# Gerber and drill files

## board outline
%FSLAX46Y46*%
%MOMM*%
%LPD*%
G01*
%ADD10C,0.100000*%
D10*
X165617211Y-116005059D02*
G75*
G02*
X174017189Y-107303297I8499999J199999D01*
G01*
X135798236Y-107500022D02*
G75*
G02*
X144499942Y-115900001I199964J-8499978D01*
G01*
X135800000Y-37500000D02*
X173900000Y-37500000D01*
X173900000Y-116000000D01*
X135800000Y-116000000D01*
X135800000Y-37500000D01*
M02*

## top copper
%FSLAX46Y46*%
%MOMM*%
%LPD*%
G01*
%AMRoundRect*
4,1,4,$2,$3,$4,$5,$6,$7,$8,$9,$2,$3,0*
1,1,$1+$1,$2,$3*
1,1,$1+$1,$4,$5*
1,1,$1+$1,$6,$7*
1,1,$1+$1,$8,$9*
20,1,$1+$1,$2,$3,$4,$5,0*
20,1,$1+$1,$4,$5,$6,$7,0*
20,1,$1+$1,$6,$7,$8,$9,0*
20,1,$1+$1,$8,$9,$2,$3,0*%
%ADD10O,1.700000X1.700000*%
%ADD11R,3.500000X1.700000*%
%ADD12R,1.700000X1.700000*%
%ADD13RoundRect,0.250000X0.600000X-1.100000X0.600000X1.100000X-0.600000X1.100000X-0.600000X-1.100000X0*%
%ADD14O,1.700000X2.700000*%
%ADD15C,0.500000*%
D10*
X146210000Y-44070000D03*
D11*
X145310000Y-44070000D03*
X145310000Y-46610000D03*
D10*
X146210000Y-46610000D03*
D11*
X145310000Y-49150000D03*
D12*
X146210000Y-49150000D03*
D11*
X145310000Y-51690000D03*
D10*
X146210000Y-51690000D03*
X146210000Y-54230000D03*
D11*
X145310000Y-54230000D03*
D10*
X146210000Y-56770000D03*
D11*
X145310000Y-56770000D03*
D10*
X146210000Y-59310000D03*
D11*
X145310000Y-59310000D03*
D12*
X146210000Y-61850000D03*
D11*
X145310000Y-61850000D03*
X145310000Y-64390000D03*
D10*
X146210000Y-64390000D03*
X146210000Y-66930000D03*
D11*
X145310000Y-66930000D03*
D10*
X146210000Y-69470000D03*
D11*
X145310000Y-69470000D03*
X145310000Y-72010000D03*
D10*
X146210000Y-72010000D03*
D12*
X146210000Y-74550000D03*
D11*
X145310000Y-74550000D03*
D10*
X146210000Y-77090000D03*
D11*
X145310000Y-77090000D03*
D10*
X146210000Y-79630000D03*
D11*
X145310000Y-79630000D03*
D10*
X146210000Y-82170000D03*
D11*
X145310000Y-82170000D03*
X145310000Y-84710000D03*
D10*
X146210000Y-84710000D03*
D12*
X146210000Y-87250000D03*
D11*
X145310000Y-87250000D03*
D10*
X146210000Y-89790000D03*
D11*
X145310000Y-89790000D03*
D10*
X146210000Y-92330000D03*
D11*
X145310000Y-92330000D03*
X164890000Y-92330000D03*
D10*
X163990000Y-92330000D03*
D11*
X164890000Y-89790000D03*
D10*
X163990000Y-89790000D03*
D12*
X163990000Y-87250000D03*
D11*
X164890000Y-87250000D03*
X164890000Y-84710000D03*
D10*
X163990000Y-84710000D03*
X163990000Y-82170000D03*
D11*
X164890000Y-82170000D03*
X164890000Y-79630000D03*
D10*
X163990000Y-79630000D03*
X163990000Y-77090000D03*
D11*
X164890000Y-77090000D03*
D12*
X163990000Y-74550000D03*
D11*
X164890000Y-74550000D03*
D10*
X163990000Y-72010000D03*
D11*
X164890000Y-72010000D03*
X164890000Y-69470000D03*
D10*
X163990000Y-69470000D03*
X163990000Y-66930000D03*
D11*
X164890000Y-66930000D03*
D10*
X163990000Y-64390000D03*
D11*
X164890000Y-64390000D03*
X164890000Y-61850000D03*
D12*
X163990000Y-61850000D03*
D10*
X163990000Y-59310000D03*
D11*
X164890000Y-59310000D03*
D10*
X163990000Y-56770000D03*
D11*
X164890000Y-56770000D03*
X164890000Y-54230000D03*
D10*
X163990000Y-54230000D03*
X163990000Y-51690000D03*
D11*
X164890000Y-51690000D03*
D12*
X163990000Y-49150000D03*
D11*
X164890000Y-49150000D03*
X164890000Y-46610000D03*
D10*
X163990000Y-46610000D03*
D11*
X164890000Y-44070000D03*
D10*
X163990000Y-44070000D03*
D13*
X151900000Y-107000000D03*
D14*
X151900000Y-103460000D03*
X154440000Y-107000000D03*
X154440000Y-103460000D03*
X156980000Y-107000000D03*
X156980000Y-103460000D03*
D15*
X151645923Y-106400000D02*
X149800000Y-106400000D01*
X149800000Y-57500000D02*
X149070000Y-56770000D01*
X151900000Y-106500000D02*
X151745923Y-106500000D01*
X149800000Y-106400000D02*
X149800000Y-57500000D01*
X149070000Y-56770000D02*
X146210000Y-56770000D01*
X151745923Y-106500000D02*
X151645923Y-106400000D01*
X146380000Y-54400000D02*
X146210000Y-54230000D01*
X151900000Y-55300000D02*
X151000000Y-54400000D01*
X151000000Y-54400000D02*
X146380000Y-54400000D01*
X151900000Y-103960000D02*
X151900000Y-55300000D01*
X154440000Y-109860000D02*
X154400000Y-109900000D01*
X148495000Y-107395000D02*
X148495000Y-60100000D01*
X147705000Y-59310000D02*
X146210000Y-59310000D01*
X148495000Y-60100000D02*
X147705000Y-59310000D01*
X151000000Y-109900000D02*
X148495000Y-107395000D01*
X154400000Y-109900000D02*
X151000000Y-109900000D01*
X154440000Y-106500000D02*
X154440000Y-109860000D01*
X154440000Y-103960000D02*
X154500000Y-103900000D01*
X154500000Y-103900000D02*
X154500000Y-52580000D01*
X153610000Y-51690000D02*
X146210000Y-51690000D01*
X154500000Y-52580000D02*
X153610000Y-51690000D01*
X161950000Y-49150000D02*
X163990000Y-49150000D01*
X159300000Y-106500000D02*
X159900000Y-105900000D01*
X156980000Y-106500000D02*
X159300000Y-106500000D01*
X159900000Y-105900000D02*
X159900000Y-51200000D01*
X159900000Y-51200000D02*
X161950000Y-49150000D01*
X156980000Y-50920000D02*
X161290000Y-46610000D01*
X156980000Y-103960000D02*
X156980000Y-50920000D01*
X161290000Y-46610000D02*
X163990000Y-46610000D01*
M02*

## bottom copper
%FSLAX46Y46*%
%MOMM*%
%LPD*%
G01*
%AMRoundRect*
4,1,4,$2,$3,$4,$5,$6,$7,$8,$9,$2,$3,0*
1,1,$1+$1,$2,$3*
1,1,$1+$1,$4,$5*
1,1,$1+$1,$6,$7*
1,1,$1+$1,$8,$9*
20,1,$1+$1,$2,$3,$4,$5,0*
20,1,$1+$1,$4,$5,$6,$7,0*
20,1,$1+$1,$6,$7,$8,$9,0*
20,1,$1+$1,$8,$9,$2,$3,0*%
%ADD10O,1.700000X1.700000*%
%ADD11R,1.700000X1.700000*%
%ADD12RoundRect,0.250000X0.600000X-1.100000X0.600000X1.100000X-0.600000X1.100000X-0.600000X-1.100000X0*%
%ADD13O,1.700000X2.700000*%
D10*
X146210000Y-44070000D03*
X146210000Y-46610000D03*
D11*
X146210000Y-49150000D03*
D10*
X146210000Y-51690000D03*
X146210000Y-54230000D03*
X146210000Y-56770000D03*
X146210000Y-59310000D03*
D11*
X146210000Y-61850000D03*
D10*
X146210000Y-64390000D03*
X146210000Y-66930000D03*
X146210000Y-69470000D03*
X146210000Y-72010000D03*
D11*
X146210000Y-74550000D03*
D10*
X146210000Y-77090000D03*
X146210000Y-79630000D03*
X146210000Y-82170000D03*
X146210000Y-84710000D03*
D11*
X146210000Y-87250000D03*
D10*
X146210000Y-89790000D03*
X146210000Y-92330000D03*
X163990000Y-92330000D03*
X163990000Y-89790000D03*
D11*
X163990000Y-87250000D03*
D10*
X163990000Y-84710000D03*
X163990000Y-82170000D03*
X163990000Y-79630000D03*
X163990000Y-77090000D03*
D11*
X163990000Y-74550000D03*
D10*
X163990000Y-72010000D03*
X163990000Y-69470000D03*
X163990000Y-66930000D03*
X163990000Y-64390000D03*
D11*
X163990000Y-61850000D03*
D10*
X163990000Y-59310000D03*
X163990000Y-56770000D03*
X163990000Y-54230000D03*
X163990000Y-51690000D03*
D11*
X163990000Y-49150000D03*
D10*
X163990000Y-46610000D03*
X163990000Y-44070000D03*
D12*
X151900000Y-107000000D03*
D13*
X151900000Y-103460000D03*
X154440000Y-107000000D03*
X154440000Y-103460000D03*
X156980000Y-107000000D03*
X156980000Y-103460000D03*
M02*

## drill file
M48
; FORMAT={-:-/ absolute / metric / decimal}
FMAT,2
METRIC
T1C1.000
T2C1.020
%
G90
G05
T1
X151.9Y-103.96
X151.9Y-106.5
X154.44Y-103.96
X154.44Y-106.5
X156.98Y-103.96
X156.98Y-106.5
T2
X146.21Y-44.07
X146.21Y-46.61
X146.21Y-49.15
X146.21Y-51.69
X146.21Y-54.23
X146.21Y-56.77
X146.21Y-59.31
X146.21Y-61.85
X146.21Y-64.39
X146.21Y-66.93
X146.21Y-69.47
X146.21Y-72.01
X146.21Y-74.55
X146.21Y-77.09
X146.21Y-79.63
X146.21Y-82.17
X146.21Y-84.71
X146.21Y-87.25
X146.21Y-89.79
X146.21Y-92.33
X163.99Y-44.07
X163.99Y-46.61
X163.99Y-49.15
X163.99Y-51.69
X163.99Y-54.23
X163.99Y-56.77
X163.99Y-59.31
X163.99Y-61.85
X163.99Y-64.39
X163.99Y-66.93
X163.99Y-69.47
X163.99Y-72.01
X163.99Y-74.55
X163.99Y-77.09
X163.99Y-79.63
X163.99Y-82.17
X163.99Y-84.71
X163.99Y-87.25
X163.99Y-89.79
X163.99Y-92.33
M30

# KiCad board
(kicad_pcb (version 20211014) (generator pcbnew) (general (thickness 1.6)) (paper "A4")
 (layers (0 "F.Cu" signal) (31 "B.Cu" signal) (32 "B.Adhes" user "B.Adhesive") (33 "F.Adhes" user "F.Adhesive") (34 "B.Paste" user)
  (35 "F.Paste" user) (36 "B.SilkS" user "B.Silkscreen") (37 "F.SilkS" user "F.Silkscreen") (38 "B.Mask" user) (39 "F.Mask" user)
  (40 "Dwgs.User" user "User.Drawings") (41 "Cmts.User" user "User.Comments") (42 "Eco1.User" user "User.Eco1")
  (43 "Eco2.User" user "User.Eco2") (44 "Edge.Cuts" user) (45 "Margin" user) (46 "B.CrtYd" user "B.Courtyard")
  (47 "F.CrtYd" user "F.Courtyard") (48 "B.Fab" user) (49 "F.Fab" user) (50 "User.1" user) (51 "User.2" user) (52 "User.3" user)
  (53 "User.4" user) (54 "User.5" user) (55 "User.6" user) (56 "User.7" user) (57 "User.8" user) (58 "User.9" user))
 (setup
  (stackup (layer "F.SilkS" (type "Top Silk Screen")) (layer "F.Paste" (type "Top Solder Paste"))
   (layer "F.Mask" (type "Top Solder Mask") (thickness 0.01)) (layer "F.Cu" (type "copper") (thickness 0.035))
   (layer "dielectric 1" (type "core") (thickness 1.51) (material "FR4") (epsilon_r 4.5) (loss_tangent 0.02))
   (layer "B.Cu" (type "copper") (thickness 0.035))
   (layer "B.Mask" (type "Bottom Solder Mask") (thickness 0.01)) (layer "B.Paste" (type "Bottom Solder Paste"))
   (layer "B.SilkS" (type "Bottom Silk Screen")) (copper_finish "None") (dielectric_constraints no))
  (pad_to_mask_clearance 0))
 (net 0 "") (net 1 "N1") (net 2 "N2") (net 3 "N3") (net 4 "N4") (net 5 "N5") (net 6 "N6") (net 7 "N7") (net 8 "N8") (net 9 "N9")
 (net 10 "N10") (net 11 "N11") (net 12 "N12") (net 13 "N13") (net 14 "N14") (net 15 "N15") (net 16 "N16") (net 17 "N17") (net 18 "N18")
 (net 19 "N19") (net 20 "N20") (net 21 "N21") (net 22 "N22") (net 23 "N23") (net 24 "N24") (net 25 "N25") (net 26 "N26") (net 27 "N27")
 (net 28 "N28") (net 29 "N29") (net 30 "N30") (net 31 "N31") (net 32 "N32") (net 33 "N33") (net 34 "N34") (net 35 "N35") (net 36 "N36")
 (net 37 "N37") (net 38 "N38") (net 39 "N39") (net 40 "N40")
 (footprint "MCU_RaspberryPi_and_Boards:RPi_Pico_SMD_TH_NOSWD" (layer "F.Cu") (at 155.1 68.2)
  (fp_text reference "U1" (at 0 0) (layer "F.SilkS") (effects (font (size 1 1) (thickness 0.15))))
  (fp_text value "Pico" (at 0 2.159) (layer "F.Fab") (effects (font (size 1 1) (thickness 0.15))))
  (pad "1" thru_hole oval (at -8.89 -24.13) (size 1.7 1.7) (drill 1.02) (layers *.Cu *.Mask) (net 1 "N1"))
  (pad "1" smd rect (at -8.89 -24.13) (size 3.5 1.7) (drill (offset -0.9 0)) (layers "F.Cu" "F.Mask") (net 1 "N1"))
  (pad "2" smd rect (at -8.89 -21.59) (size 3.5 1.7) (drill (offset -0.9 0)) (layers "F.Cu" "F.Mask") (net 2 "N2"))
  (pad "2" thru_hole oval (at -8.89 -21.59) (size 1.7 1.7) (drill 1.02) (layers *.Cu *.Mask) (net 2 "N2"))
  (pad "3" smd rect (at -8.89 -19.05) (size 3.5 1.7) (drill (offset -0.9 0)) (layers "F.Cu" "F.Mask") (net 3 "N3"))
  (pad "3" thru_hole rect (at -8.89 -19.05) (size 1.7 1.7) (drill 1.02) (layers *.Cu *.Mask) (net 3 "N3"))
  (pad "4" smd rect (at -8.89 -16.51) (size 3.5 1.7) (drill (offset -0.9 0)) (layers "F.Cu" "F.Mask") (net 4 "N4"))
  (pad "4" thru_hole oval (at -8.89 -16.51) (size 1.7 1.7) (drill 1.02) (layers *.Cu *.Mask) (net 4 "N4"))
  (pad "5" thru_hole oval (at -8.89 -13.97) (size 1.7 1.7) (drill 1.02) (layers *.Cu *.Mask) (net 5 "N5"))
  (pad "5" smd rect (at -8.89 -13.97) (size 3.5 1.7) (drill (offset -0.9 0)) (layers "F.Cu" "F.Mask") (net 5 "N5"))
  (pad "6" thru_hole oval (at -8.89 -11.43) (size 1.7 1.7) (drill 1.02) (layers *.Cu *.Mask) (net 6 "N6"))
  (pad "6" smd rect (at -8.89 -11.43) (size 3.5 1.7) (drill (offset -0.9 0)) (layers "F.Cu" "F.Mask") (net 6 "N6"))
  (pad "7" thru_hole oval (at -8.89 -8.89) (size 1.7 1.7) (drill 1.02) (layers *.Cu *.Mask) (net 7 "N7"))
  (pad "7" smd rect (at -8.89 -8.89) (size 3.5 1.7) (drill (offset -0.9 0)) (layers "F.Cu" "F.Mask") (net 7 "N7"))
  (pad "8" thru_hole rect (at -8.89 -6.35) (size 1.7 1.7) (drill 1.02) (layers *.Cu *.Mask) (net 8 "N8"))
  (pad "8" smd rect (at -8.89 -6.35) (size 3.5 1.7) (drill (offset -0.9 0)) (layers "F.Cu" "F.Mask") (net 8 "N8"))
  (pad "9" smd rect (at -8.89 -3.81) (size 3.5 1.7) (drill (offset -0.9 0)) (layers "F.Cu" "F.Mask") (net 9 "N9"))
  (pad "9" thru_hole oval (at -8.89 -3.81) (size 1.7 1.7) (drill 1.02) (layers *.Cu *.Mask) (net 9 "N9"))
  (pad "10" thru_hole oval (at -8.89 -1.27) (size 1.7 1.7) (drill 1.02) (layers *.Cu *.Mask) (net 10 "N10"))
  (pad "10" smd rect (at -8.89 -1.27) (size 3.5 1.7) (drill (offset -0.9 0)) (layers "F.Cu" "F.Mask") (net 10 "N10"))
  (pad "11" thru_hole oval (at -8.89 1.27) (size 1.7 1.7) (drill 1.02) (layers *.Cu *.Mask) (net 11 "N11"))
  (pad "11" smd rect (at -8.89 1.27) (size 3.5 1.7) (drill (offset -0.9 0)) (layers "F.Cu" "F.Mask") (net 11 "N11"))
  (pad "12" smd rect (at -8.89 3.81) (size 3.5 1.7) (drill (offset -0.9 0)) (layers "F.Cu" "F.Mask") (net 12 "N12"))
  (pad "12" thru_hole oval (at -8.89 3.81) (size 1.7 1.7) (drill 1.02) (layers *.Cu *.Mask) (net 12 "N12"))
  (pad "13" thru_hole rect (at -8.89 6.35) (size 1.7 1.7) (drill 1.02) (layers *.Cu *.Mask) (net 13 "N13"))
  (pad "13" smd rect (at -8.89 6.35) (size 3.5 1.7) (drill (offset -0.9 0)) (layers "F.Cu" "F.Mask") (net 13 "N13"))
  (pad "14" thru_hole oval (at -8.89 8.89) (size 1.7 1.7) (drill 1.02) (layers *.Cu *.Mask) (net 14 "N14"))
  (pad "14" smd rect (at -8.89 8.89) (size 3.5 1.7) (drill (offset -0.9 0)) (layers "F.Cu" "F.Mask") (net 14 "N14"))
  (pad "15" thru_hole oval (at -8.89 11.43) (size 1.7 1.7) (drill 1.02) (layers *.Cu *.Mask) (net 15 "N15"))
  (pad "15" smd rect (at -8.89 11.43) (size 3.5 1.7) (drill (offset -0.9 0)) (layers "F.Cu" "F.Mask") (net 15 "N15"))
  (pad "16" thru_hole oval (at -8.89 13.97) (size 1.7 1.7) (drill 1.02) (layers *.Cu *.Mask) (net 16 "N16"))
  (pad "16" smd rect (at -8.89 13.97) (size 3.5 1.7) (drill (offset -0.9 0)) (layers "F.Cu" "F.Mask") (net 16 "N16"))
  (pad "17" smd rect (at -8.89 16.51) (size 3.5 1.7) (drill (offset -0.9 0)) (layers "F.Cu" "F.Mask") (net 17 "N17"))
  (pad "17" thru_hole oval (at -8.89 16.51) (size 1.7 1.7) (drill 1.02) (layers *.Cu *.Mask) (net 17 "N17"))
  (pad "18" thru_hole rect (at -8.89 19.05) (size 1.7 1.7) (drill 1.02) (layers *.Cu *.Mask) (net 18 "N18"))
  (pad "18" smd rect (at -8.89 19.05) (size 3.5 1.7) (drill (offset -0.9 0)) (layers "F.Cu" "F.Mask") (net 18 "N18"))
  (pad "19" thru_hole oval (at -8.89 21.59) (size 1.7 1.7) (drill 1.02) (layers *.Cu *.Mask) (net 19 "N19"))
  (pad "19" smd rect (at -8.89 21.59) (size 3.5 1.7) (drill (offset -0.9 0)) (layers "F.Cu" "F.Mask") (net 19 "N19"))
  (pad "20" thru_hole oval (at -8.89 24.13) (size 1.7 1.7) (drill 1.02) (layers *.Cu *.Mask) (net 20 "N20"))
  (pad "20" smd rect (at -8.89 24.13) (size 3.5 1.7) (drill (offset -0.9 0)) (layers "F.Cu" "F.Mask") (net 20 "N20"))
  (pad "21" smd rect (at 8.89 24.13) (size 3.5 1.7) (drill (offset 0.9 0)) (layers "F.Cu" "F.Mask") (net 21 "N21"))
  (pad "21" thru_hole oval (at 8.89 24.13) (size 1.7 1.7) (drill 1.02) (layers *.Cu *.Mask) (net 21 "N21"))
  (pad "22" smd rect (at 8.89 21.59) (size 3.5 1.7) (drill (offset 0.9 0)) (layers "F.Cu" "F.Mask") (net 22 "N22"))
  (pad "22" thru_hole oval (at 8.89 21.59) (size 1.7 1.7) (drill 1.02) (layers *.Cu *.Mask) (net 22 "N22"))
  (pad "23" thru_hole rect (at 8.89 19.05) (size 1.7 1.7) (drill 1.02) (layers *.Cu *.Mask) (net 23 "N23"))
  (pad "23" smd rect (at 8.89 19.05) (size 3.5 1.7) (drill (offset 0.9 0)) (layers "F.Cu" "F.Mask") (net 23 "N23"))
  (pad "24" smd rect (at 8.89 16.51) (size 3.5 1.7) (drill (offset 0.9 0)) (layers "F.Cu" "F.Mask") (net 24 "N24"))
  (pad "24" thru_hole oval (at 8.89 16.51) (size 1.7 1.7) (drill 1.02) (layers *.Cu *.Mask) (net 24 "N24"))
  (pad "25" thru_hole oval (at 8.89 13.97) (size 1.7 1.7) (drill 1.02) (layers *.Cu *.Mask) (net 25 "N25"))
  (pad "25" smd rect (at 8.89 13.97) (size 3.5 1.7) (drill (offset 0.9 0)) (layers "F.Cu" "F.Mask") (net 25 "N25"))
  (pad "26" smd rect (at 8.89 11.43) (size 3.5 1.7) (drill (offset 0.9 0)) (layers "F.Cu" "F.Mask") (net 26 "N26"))
  (pad "26" thru_hole oval (at 8.89 11.43) (size 1.7 1.7) (drill 1.02) (layers *.Cu *.Mask) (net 26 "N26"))
  (pad "27" thru_hole oval (at 8.89 8.89) (size 1.7 1.7) (drill 1.02) (layers *.Cu *.Mask) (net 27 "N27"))
  (pad "27" smd rect (at 8.89 8.89) (size 3.5 1.7) (drill (offset 0.9 0)) (layers "F.Cu" "F.Mask") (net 27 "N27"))
  (pad "28" thru_hole rect (at 8.89 6.35) (size 1.7 1.7) (drill 1.02) (layers *.Cu *.Mask) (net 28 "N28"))
  (pad "28" smd rect (at 8.89 6.35) (size 3.5 1.7) (drill (offset 0.9 0)) (layers "F.Cu" "F.Mask") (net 28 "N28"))
  (pad "29" thru_hole oval (at 8.89 3.81) (size 1.7 1.7) (drill 1.02) (layers *.Cu *.Mask) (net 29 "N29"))
  (pad "29" smd rect (at 8.89 3.81) (size 3.5 1.7) (drill (offset 0.9 0)) (layers "F.Cu" "F.Mask") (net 29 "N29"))
  (pad "30" smd rect (at 8.89 1.27) (size 3.5 1.7) (drill (offset 0.9 0)) (layers "F.Cu" "F.Mask") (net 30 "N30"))
  (pad "30" thru_hole oval (at 8.89 1.27) (size 1.7 1.7) (drill 1.02) (layers *.Cu *.Mask) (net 30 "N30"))
  (pad "31" thru_hole oval (at 8.89 -1.27) (size 1.7 1.7) (drill 1.02) (layers *.Cu *.Mask) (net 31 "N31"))
  (pad "31" smd rect (at 8.89 -1.27) (size 3.5 1.7) (drill (offset 0.9 0)) (layers "F.Cu" "F.Mask") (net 31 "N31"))
  (pad "32" thru_hole oval (at 8.89 -3.81) (size 1.7 1.7) (drill 1.02) (layers *.Cu *.Mask) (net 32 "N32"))
  (pad "32" smd rect (at 8.89 -3.81) (size 3.5 1.7) (drill (offset 0.9 0)) (layers "F.Cu" "F.Mask") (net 32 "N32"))
  (pad "33" smd rect (at 8.89 -6.35) (size 3.5 1.7) (drill (offset 0.9 0)) (layers "F.Cu" "F.Mask") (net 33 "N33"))
  (pad "33" thru_hole rect (at 8.89 -6.35) (size 1.7 1.7) (drill 1.02) (layers *.Cu *.Mask) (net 33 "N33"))
  (pad "34" thru_hole oval (at 8.89 -8.89) (size 1.7 1.7) (drill 1.02) (layers *.Cu *.Mask) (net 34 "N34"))
  (pad "34" smd rect (at 8.89 -8.89) (size 3.5 1.7) (drill (offset 0.9 0)) (layers "F.Cu" "F.Mask") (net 34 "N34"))
  (pad "35" thru_hole oval (at 8.89 -11.43) (size 1.7 1.7) (drill 1.02) (layers *.Cu *.Mask) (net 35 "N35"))
  (pad "35" smd rect (at 8.89 -11.43) (size 3.5 1.7) (drill (offset 0.9 0)) (layers "F.Cu" "F.Mask") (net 35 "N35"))
  (pad "36" smd rect (at 8.89 -13.97) (size 3.5 1.7) (drill (offset 0.9 0)) (layers "F.Cu" "F.Mask") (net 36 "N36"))
  (pad "36" thru_hole oval (at 8.89 -13.97) (size 1.7 1.7) (drill 1.02) (layers *.Cu *.Mask) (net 36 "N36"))
  (pad "37" thru_hole oval (at 8.89 -16.51) (size 1.7 1.7) (drill 1.02) (layers *.Cu *.Mask) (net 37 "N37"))
  (pad "37" smd rect (at 8.89 -16.51) (size 3.5 1.7) (drill (offset 0.9 0)) (layers "F.Cu" "F.Mask") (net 37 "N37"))
  (pad "38" thru_hole rect (at 8.89 -19.05) (size 1.7 1.7) (drill 1.02) (layers *.Cu *.Mask) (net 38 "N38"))
  (pad "38" smd rect (at 8.89 -19.05) (size 3.5 1.7) (drill (offset 0.9 0)) (layers "F.Cu" "F.Mask") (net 38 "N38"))
  (pad "39" smd rect (at 8.89 -21.59) (size 3.5 1.7) (drill (offset 0.9 0)) (layers "F.Cu" "F.Mask") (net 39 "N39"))
  (pad "39" thru_hole oval (at 8.89 -21.59) (size 1.7 1.7) (drill 1.02) (layers *.Cu *.Mask) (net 39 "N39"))
  (pad "40" smd rect (at 8.89 -24.13) (size 3.5 1.7) (drill (offset 0.9 0)) (layers "F.Cu" "F.Mask") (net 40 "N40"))
  (pad "40" thru_hole oval (at 8.89 -24.13) (size 1.7 1.7) (drill 1.02) (layers *.Cu *.Mask) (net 40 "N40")))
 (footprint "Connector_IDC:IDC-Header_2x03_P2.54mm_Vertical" (layer "F.Cu") (at 151.9 106.5 90)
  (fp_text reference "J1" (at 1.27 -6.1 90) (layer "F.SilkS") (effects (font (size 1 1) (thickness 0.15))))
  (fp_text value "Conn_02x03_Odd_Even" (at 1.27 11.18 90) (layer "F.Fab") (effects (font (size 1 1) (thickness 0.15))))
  (pad "1" thru_hole roundrect (at 0 0 90) (size 2.7 1.7) (drill 1 (offset -0.5 0)) (layers *.Cu *.Mask) (roundrect_rratio 0.1470588235)
   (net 6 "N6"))
  (pad "2" thru_hole oval (at 2.54 0 90) (size 2.7 1.7) (drill 1 (offset 0.5 0)) (layers *.Cu *.Mask) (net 5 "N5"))
  (pad "3" thru_hole oval (at 0 2.54 90) (size 2.7 1.7) (drill 1 (offset -0.5 0)) (layers *.Cu *.Mask) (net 7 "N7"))
  (pad "4" thru_hole oval (at 2.54 2.54 90) (size 2.7 1.7) (drill 1 (offset 0.5 0)) (layers *.Cu *.Mask) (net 4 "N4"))
  (pad "5" thru_hole oval (at 0 5.08 90) (size 2.7 1.7) (drill 1 (offset -0.5 0)) (layers *.Cu *.Mask) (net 38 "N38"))
  (pad "6" thru_hole oval (at 2.54 5.08 90) (size 2.7 1.7) (drill 1 (offset 0.5 0)) (layers *.Cu *.Mask) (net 39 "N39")))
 (gr_arc (start 165.617211 116.005059) (mid 168 109.9) (end 174.017189 107.303295) (layer "Edge.Cuts") (width 0.1))
 (gr_arc (start 135.798236 107.500022) (mid 141.903295 109.882811) (end 144.5 115.9) (layer "Edge.Cuts") (width 0.1))
 (gr_rect (start 135.8 37.5) (end 173.9 116) (layer "Edge.Cuts") (width 0.1) (fill none))
 (segment (start 151.645923 106.4) (end 149.8 106.4) (width 0.5) (layer "F.Cu") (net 6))
 (segment (start 149.8 57.5) (end 149.07 56.77) (width 0.5) (layer "F.Cu") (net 6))
 (segment (start 151.9 106.5) (end 151.745923 106.5) (width 0.5) (layer "F.Cu") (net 6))
 (segment (start 149.8 106.4) (end 149.8 57.5) (width 0.5) (layer "F.Cu") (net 6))
 (segment (start 149.07 56.77) (end 146.21 56.77) (width 0.5) (layer "F.Cu") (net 6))
 (segment (start 151.745923 106.5) (end 151.645923 106.4) (width 0.5) (layer "F.Cu") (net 6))
 (segment (start 146.38 54.4) (end 146.21 54.23) (width 0.5) (layer "F.Cu") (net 5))
 (segment (start 151.9 55.3) (end 151 54.4) (width 0.5) (layer "F.Cu") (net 5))
 (segment (start 151 54.4) (end 146.38 54.4) (width 0.5) (layer "F.Cu") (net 5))
 (segment (start 151.9 103.96) (end 151.9 55.3) (width 0.5) (layer "F.Cu") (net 5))
 (segment (start 154.44 109.86) (end 154.4 109.9) (width 0.5) (layer "F.Cu") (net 7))
 (segment (start 148.495 107.395) (end 148.495 60.1) (width 0.5) (layer "F.Cu") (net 7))
 (segment (start 147.705 59.31) (end 146.21 59.31) (width 0.5) (layer "F.Cu") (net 7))
 (segment (start 148.495 60.1) (end 147.705 59.31) (width 0.5) (layer "F.Cu") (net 7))
 (segment (start 151 109.9) (end 148.495 107.395) (width 0.5) (layer "F.Cu") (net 7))
 (segment (start 154.4 109.9) (end 151 109.9) (width 0.5) (layer "F.Cu") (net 7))
 (segment (start 154.44 106.5) (end 154.44 109.86) (width 0.5) (layer "F.Cu") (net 7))
 (segment (start 154.44 103.96) (end 154.5 103.9) (width 0.5) (layer "F.Cu") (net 4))
 (segment (start 154.5 103.9) (end 154.5 52.58) (width 0.5) (layer "F.Cu") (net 4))
 (segment (start 153.61 51.69) (end 146.21 51.69) (width 0.5) (layer "F.Cu") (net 4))
 (segment (start 154.5 52.58) (end 153.61 51.69) (width 0.5) (layer "F.Cu") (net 4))
 (segment (start 161.95 49.15) (end 163.99 49.15) (width 0.5) (layer "F.Cu") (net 38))
 (segment (start 159.3 106.5) (end 159.9 105.9) (width 0.5) (layer "F.Cu") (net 38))
 (segment (start 156.98 106.5) (end 159.3 106.5) (width 0.5) (layer "F.Cu") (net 38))
 (segment (start 159.9 105.9) (end 159.9 51.2) (width 0.5) (layer "F.Cu") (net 38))
 (segment (start 159.9 51.2) (end 161.95 49.15) (width 0.5) (layer "F.Cu") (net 38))
 (segment (start 156.98 50.92) (end 161.29 46.61) (width 0.5) (layer "F.Cu") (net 39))
 (segment (start 156.98 103.96) (end 156.98 50.92) (width 0.5) (layer "F.Cu") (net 39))
 (segment (start 161.29 46.61) (end 163.99 46.61) (width 0.5) (layer "F.Cu") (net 39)))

